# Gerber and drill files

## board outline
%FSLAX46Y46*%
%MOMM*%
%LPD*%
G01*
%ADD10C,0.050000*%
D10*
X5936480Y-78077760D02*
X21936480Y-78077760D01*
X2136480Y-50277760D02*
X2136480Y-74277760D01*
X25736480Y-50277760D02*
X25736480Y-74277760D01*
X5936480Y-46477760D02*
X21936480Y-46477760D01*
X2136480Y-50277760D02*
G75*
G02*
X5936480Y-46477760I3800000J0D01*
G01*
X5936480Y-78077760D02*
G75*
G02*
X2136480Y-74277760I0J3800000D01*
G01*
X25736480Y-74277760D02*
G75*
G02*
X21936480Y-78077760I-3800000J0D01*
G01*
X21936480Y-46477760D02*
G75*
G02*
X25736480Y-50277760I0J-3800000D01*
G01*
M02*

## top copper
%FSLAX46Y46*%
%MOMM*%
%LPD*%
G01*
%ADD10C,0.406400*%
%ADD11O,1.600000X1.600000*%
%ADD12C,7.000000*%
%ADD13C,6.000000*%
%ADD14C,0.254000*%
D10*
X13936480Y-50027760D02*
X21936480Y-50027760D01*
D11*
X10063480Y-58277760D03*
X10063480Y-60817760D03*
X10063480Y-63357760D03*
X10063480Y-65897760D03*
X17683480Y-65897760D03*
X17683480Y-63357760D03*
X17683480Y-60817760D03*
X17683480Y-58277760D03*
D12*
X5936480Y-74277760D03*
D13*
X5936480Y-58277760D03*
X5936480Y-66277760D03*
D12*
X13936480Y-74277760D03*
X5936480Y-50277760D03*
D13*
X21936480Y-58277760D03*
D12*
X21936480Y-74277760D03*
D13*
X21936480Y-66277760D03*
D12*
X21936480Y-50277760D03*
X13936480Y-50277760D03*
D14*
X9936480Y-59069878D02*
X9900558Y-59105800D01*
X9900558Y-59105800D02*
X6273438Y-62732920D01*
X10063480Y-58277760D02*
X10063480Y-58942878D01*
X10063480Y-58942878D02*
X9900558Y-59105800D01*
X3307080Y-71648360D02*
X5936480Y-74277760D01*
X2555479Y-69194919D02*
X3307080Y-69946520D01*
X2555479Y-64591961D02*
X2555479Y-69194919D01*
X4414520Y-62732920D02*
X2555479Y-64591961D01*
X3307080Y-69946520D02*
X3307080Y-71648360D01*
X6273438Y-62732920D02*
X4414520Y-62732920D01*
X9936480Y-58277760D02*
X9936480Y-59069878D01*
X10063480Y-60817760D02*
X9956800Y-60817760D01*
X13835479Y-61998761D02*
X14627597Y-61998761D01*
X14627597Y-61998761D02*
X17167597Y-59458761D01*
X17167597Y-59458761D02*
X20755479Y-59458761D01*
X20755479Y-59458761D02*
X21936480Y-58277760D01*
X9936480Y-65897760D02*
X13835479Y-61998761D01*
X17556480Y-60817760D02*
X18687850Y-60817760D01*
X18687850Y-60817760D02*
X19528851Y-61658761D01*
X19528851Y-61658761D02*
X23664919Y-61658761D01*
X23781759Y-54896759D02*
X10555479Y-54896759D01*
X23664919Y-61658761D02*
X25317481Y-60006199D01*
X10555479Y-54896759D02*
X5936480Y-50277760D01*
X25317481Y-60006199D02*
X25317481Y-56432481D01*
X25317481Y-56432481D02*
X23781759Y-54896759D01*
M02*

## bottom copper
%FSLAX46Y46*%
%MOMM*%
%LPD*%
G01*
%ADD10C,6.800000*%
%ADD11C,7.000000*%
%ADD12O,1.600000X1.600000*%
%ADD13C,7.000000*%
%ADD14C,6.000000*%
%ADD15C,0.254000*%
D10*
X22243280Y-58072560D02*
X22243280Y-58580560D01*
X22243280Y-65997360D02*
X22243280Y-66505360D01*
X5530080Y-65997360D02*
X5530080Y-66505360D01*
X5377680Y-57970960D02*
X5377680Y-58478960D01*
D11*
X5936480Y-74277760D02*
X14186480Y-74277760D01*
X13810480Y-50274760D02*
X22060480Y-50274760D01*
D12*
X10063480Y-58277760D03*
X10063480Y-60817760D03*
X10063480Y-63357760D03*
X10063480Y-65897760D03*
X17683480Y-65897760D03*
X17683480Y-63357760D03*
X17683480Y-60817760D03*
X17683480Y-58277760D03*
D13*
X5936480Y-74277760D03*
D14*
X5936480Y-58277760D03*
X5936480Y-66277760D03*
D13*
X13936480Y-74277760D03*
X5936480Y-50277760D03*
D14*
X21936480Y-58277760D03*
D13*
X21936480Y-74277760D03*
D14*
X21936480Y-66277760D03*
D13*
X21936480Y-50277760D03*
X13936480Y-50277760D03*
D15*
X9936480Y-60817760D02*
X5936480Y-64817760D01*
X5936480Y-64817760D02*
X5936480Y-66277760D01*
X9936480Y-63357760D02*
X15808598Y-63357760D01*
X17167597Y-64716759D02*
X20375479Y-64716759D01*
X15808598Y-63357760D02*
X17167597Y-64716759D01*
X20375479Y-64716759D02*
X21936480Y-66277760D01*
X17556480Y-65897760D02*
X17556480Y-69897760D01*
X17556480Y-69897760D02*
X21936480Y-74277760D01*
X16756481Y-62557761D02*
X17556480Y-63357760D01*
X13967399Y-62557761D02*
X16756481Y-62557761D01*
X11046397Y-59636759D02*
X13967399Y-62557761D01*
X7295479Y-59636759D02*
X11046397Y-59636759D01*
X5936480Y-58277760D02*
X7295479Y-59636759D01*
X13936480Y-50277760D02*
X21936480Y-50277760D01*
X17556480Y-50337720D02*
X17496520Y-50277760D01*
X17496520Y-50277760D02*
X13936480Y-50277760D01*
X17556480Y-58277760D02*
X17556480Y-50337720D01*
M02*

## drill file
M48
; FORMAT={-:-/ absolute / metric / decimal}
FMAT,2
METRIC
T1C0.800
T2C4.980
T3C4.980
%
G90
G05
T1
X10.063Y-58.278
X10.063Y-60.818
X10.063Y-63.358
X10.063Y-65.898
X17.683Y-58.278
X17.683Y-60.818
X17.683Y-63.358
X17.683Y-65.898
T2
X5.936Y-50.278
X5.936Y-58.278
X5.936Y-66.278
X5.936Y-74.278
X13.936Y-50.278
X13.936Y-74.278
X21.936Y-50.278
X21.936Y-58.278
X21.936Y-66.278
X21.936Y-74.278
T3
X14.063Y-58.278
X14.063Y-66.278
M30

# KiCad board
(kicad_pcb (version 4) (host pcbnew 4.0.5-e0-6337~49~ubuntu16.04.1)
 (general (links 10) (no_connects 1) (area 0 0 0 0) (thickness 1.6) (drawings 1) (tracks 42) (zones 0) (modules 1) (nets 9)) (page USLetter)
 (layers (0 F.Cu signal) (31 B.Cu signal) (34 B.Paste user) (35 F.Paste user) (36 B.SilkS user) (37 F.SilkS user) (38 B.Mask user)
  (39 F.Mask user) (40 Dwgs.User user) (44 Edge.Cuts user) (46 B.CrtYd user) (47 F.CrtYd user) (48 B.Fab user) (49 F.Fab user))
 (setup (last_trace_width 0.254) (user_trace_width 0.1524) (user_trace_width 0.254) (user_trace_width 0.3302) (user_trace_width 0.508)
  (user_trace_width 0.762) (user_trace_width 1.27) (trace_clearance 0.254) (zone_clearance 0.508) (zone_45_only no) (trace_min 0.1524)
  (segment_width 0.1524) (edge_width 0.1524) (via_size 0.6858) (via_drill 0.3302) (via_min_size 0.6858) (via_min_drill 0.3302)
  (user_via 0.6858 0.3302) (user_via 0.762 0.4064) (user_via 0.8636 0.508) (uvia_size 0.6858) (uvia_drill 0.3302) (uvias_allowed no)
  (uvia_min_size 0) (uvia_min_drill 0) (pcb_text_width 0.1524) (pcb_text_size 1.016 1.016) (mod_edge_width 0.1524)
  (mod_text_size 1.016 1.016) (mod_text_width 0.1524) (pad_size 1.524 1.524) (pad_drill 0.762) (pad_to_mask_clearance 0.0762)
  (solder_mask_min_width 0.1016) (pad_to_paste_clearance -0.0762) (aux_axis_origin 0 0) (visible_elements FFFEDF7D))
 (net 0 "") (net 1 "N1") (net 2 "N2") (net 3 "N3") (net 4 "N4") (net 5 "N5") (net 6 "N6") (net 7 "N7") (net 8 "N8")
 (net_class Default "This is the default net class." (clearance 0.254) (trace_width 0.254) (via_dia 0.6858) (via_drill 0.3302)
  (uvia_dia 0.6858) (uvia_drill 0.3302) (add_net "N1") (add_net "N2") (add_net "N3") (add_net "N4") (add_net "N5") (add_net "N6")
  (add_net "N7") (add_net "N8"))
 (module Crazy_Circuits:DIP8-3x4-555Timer (layer F.Cu) (at 5.93648 74.27776)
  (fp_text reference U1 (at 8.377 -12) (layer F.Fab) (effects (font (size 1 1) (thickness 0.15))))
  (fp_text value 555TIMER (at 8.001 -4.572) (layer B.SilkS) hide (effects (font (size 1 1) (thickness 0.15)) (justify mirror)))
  (fp_line (start 16.3068 -16.2052) (end 16.3068 -15.6972) (layer B.Cu) (width 6.8))
  (fp_line (start 8 -24.25) (end 16 -24.25) (layer F.Cu) (width 0.4064))
  (fp_line (start 0 3.8) (end 16 3.8) (layer Edge.Cuts) (width 0.05))
  (fp_line (start -3.8 -24) (end -3.8 0) (layer Edge.Cuts) (width 0.05))
  (fp_line (start 19.8 -24) (end 19.8 0) (layer Edge.Cuts) (width 0.05))
  (fp_line (start 0 -27.8) (end 16 -27.8) (layer Edge.Cuts) (width 0.05))
  (fp_arc (start 0 -24) (end -3.8 -24) (angle 90) (layer Edge.Cuts) (width 0.05))
  (fp_arc (start 0 0) (end 0 3.8) (angle 90) (layer Edge.Cuts) (width 0.05))
  (fp_arc (start 16 0) (end 19.8 0) (angle 90) (layer Edge.Cuts) (width 0.05))
  (fp_arc (start 16 -24) (end 16 -27.8) (angle 90) (layer Edge.Cuts) (width 0.05))
  (fp_line (start 16.3068 -8.2804) (end 16.3068 -7.7724) (layer B.Cu) (width 6.8))
  (fp_line (start -0.4064 -8.2804) (end -0.4064 -7.7724) (layer B.Cu) (width 6.8))
  (fp_line (start -0.5588 -16.3068) (end -0.5588 -15.7988) (layer B.Cu) (width 6.8))
  (fp_line (start 0 0) (end 8.25 0) (layer B.Cu) (width 7))
  (fp_line (start 7.874 -24.003) (end 16.124 -24.003) (layer B.Cu) (width 7))
  (pad 1 thru_hole oval (at 4.127 -16) (size 1.6 1.6) (drill 0.8) (layers *.Cu *.Mask F.SilkS) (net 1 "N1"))
  (pad 2 thru_hole oval (at 4.127 -13.46) (size 1.6 1.6) (drill 0.8) (layers *.Cu *.Mask F.SilkS) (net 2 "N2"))
  (pad 3 thru_hole oval (at 4.127 -10.92) (size 1.6 1.6) (drill 0.8) (layers *.Cu *.Mask F.SilkS) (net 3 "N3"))
  (pad 4 thru_hole oval (at 4.127 -8.38) (size 1.6 1.6) (drill 0.8) (layers *.Cu *.Mask F.SilkS) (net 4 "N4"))
  (pad 5 thru_hole oval (at 11.747 -8.38) (size 1.6 1.6) (drill 0.8) (layers *.Cu *.Mask F.SilkS) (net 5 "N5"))
  (pad 6 thru_hole oval (at 11.747 -10.92) (size 1.6 1.6) (drill 0.8) (layers *.Cu *.Mask F.SilkS) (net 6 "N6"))
  (pad 7 thru_hole oval (at 11.747 -13.46) (size 1.6 1.6) (drill 0.8) (layers *.Cu *.Mask F.SilkS) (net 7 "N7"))
  (pad 8 thru_hole oval (at 11.747 -16) (size 1.6 1.6) (drill 0.8) (layers *.Cu *.Mask F.SilkS) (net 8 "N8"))
  (pad 1 thru_hole circle (at 0 0 270) (size 7 7) (drill 4.98) (layers *.Cu B.Mask) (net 1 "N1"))
  (pad "" np_thru_hole circle (at 8.127 -16 270) (size 4.98 4.98) (drill 4.98) (layers *.Cu))
  (pad 6 thru_hole circle (at 0 -16 270) (size 6 6) (drill 4.98) (layers *.Cu B.Mask) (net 6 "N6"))
  (pad 2 thru_hole circle (at 0 -8 270) (size 6 6) (drill 4.98) (layers *.Cu B.Mask) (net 2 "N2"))
  (pad "" np_thru_hole circle (at 8.127 -8 270) (size 4.98 4.98) (drill 4.98) (layers *.Cu F.SilkS))
  (pad 1 thru_hole circle (at 8 0 270) (size 7 7) (drill 4.98) (layers *.Cu B.Mask) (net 1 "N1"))
  (pad 7 thru_hole circle (at 0 -24 270) (size 7 7) (drill 4.98) (layers *.Cu B.Mask) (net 7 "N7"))
  (pad 4 thru_hole circle (at 16 -16 270) (size 6 6) (drill 4.98) (layers *.Cu B.Mask) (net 4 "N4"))
  (pad 5 thru_hole circle (at 16 0 270) (size 7 7) (drill 4.98) (layers *.Cu B.Mask) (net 5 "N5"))
  (pad 3 thru_hole circle (at 16 -8 270) (size 6 6) (drill 4.98) (layers *.Cu B.Mask) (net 3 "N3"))
  (pad 8 thru_hole circle (at 16 -24 270) (size 7 7) (drill 4.98) (layers *.Cu B.Mask) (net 8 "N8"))
  (pad 8 thru_hole circle (at 8 -24 270) (size 7 7) (drill 4.98) (layers *.Cu B.Mask) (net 8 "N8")))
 (segment (start 9.93648 59.069878) (end 9.900558 59.1058) (width 0.254) (layer F.Cu) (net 1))
 (segment (start 9.900558 59.1058) (end 6.273438 62.73292) (width 0.254) (layer F.Cu) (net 1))
 (segment (start 10.06348 58.27776) (end 10.06348 58.942878) (width 0.254) (layer F.Cu) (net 1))
 (segment (start 10.06348 58.942878) (end 9.900558 59.1058) (width 0.254) (layer F.Cu) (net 1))
 (segment (start 3.30708 71.64836) (end 5.93648 74.27776) (width 0.254) (layer F.Cu) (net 1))
 (segment (start 2.555479 69.194919) (end 3.30708 69.94652) (width 0.254) (layer F.Cu) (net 1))
 (segment (start 2.555479 64.591961) (end 2.555479 69.194919) (width 0.254) (layer F.Cu) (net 1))
 (segment (start 4.41452 62.73292) (end 2.555479 64.591961) (width 0.254) (layer F.Cu) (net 1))
 (segment (start 3.30708 69.94652) (end 3.30708 71.64836) (width 0.254) (layer F.Cu) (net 1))
 (segment (start 6.273438 62.73292) (end 4.41452 62.73292) (width 0.254) (layer F.Cu) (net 1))
 (segment (start 9.93648 58.27776) (end 9.93648 59.069878) (width 0.254) (layer F.Cu) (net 1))
 (segment (start 9.93648 60.81776) (end 5.93648 64.81776) (width 0.254) (layer B.Cu) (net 2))
 (segment (start 10.06348 60.81776) (end 9.9568 60.81776) (width 0.254) (layer F.Cu) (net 2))
 (segment (start 5.93648 64.81776) (end 5.93648 66.27776) (width 0.254) (layer B.Cu) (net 2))
 (segment (start 9.93648 63.35776) (end 15.808598 63.35776) (width 0.254) (layer B.Cu) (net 3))
 (segment (start 17.167597 64.716759) (end 20.375479 64.716759) (width 0.254) (layer B.Cu) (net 3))
 (segment (start 15.808598 63.35776) (end 17.167597 64.716759) (width 0.254) (layer B.Cu) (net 3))
 (segment (start 20.375479 64.716759) (end 21.93648 66.27776) (width 0.254) (layer B.Cu) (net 3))
 (segment (start 13.835479 61.998761) (end 14.627597 61.998761) (width 0.254) (layer F.Cu) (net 4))
 (segment (start 14.627597 61.998761) (end 17.167597 59.458761) (width 0.254) (layer F.Cu) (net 4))
 (segment (start 17.167597 59.458761) (end 20.755479 59.458761) (width 0.254) (layer F.Cu) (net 4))
 (segment (start 20.755479 59.458761) (end 21.93648 58.27776) (width 0.254) (layer F.Cu) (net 4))
 (segment (start 9.93648 65.89776) (end 13.835479 61.998761) (width 0.254) (layer F.Cu) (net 4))
 (segment (start 17.55648 65.89776) (end 17.55648 69.89776) (width 0.254) (layer B.Cu) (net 5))
 (segment (start 17.55648 69.89776) (end 21.93648 74.27776) (width 0.254) (layer B.Cu) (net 5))
 (segment (start 16.756481 62.557761) (end 17.55648 63.35776) (width 0.254) (layer B.Cu) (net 6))
 (segment (start 13.967399 62.557761) (end 16.756481 62.557761) (width 0.254) (layer B.Cu) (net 6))
 (segment (start 11.046397 59.636759) (end 13.967399 62.557761) (width 0.254) (layer B.Cu) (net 6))
 (segment (start 7.295479 59.636759) (end 11.046397 59.636759) (width 0.254) (layer B.Cu) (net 6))
 (segment (start 5.93648 58.27776) (end 7.295479 59.636759) (width 0.254) (layer B.Cu) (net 6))
 (segment (start 17.55648 60.81776) (end 18.68785 60.81776) (width 0.254) (layer F.Cu) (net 7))
 (segment (start 18.68785 60.81776) (end 19.528851 61.658761) (width 0.254) (layer F.Cu) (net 7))
 (segment (start 19.528851 61.658761) (end 23.664919 61.658761) (width 0.254) (layer F.Cu) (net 7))
 (segment (start 23.781759 54.896759) (end 10.555479 54.896759) (width 0.254) (layer F.Cu) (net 7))
 (segment (start 23.664919 61.658761) (end 25.317481 60.006199) (width 0.254) (layer F.Cu) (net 7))
 (segment (start 10.555479 54.896759) (end 5.93648 50.27776) (width 0.254) (layer F.Cu) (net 7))
 (segment (start 25.317481 60.006199) (end 25.317481 56.432481) (width 0.254) (layer F.Cu) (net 7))
 (segment (start 25.317481 56.432481) (end 23.781759 54.896759) (width 0.254) (layer F.Cu) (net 7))
 (segment (start 13.93648 50.27776) (end 21.93648 50.27776) (width 0.254) (layer B.Cu) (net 8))
 (segment (start 17.55648 50.33772) (end 17.49652 50.27776) (width 0.254) (layer B.Cu) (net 8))
 (segment (start 17.49652 50.27776) (end 13.93648 50.27776) (width 0.254) (layer B.Cu) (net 8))
 (segment (start 17.55648 58.27776) (end 17.55648 50.33772) (width 0.254) (layer B.Cu) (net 8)))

